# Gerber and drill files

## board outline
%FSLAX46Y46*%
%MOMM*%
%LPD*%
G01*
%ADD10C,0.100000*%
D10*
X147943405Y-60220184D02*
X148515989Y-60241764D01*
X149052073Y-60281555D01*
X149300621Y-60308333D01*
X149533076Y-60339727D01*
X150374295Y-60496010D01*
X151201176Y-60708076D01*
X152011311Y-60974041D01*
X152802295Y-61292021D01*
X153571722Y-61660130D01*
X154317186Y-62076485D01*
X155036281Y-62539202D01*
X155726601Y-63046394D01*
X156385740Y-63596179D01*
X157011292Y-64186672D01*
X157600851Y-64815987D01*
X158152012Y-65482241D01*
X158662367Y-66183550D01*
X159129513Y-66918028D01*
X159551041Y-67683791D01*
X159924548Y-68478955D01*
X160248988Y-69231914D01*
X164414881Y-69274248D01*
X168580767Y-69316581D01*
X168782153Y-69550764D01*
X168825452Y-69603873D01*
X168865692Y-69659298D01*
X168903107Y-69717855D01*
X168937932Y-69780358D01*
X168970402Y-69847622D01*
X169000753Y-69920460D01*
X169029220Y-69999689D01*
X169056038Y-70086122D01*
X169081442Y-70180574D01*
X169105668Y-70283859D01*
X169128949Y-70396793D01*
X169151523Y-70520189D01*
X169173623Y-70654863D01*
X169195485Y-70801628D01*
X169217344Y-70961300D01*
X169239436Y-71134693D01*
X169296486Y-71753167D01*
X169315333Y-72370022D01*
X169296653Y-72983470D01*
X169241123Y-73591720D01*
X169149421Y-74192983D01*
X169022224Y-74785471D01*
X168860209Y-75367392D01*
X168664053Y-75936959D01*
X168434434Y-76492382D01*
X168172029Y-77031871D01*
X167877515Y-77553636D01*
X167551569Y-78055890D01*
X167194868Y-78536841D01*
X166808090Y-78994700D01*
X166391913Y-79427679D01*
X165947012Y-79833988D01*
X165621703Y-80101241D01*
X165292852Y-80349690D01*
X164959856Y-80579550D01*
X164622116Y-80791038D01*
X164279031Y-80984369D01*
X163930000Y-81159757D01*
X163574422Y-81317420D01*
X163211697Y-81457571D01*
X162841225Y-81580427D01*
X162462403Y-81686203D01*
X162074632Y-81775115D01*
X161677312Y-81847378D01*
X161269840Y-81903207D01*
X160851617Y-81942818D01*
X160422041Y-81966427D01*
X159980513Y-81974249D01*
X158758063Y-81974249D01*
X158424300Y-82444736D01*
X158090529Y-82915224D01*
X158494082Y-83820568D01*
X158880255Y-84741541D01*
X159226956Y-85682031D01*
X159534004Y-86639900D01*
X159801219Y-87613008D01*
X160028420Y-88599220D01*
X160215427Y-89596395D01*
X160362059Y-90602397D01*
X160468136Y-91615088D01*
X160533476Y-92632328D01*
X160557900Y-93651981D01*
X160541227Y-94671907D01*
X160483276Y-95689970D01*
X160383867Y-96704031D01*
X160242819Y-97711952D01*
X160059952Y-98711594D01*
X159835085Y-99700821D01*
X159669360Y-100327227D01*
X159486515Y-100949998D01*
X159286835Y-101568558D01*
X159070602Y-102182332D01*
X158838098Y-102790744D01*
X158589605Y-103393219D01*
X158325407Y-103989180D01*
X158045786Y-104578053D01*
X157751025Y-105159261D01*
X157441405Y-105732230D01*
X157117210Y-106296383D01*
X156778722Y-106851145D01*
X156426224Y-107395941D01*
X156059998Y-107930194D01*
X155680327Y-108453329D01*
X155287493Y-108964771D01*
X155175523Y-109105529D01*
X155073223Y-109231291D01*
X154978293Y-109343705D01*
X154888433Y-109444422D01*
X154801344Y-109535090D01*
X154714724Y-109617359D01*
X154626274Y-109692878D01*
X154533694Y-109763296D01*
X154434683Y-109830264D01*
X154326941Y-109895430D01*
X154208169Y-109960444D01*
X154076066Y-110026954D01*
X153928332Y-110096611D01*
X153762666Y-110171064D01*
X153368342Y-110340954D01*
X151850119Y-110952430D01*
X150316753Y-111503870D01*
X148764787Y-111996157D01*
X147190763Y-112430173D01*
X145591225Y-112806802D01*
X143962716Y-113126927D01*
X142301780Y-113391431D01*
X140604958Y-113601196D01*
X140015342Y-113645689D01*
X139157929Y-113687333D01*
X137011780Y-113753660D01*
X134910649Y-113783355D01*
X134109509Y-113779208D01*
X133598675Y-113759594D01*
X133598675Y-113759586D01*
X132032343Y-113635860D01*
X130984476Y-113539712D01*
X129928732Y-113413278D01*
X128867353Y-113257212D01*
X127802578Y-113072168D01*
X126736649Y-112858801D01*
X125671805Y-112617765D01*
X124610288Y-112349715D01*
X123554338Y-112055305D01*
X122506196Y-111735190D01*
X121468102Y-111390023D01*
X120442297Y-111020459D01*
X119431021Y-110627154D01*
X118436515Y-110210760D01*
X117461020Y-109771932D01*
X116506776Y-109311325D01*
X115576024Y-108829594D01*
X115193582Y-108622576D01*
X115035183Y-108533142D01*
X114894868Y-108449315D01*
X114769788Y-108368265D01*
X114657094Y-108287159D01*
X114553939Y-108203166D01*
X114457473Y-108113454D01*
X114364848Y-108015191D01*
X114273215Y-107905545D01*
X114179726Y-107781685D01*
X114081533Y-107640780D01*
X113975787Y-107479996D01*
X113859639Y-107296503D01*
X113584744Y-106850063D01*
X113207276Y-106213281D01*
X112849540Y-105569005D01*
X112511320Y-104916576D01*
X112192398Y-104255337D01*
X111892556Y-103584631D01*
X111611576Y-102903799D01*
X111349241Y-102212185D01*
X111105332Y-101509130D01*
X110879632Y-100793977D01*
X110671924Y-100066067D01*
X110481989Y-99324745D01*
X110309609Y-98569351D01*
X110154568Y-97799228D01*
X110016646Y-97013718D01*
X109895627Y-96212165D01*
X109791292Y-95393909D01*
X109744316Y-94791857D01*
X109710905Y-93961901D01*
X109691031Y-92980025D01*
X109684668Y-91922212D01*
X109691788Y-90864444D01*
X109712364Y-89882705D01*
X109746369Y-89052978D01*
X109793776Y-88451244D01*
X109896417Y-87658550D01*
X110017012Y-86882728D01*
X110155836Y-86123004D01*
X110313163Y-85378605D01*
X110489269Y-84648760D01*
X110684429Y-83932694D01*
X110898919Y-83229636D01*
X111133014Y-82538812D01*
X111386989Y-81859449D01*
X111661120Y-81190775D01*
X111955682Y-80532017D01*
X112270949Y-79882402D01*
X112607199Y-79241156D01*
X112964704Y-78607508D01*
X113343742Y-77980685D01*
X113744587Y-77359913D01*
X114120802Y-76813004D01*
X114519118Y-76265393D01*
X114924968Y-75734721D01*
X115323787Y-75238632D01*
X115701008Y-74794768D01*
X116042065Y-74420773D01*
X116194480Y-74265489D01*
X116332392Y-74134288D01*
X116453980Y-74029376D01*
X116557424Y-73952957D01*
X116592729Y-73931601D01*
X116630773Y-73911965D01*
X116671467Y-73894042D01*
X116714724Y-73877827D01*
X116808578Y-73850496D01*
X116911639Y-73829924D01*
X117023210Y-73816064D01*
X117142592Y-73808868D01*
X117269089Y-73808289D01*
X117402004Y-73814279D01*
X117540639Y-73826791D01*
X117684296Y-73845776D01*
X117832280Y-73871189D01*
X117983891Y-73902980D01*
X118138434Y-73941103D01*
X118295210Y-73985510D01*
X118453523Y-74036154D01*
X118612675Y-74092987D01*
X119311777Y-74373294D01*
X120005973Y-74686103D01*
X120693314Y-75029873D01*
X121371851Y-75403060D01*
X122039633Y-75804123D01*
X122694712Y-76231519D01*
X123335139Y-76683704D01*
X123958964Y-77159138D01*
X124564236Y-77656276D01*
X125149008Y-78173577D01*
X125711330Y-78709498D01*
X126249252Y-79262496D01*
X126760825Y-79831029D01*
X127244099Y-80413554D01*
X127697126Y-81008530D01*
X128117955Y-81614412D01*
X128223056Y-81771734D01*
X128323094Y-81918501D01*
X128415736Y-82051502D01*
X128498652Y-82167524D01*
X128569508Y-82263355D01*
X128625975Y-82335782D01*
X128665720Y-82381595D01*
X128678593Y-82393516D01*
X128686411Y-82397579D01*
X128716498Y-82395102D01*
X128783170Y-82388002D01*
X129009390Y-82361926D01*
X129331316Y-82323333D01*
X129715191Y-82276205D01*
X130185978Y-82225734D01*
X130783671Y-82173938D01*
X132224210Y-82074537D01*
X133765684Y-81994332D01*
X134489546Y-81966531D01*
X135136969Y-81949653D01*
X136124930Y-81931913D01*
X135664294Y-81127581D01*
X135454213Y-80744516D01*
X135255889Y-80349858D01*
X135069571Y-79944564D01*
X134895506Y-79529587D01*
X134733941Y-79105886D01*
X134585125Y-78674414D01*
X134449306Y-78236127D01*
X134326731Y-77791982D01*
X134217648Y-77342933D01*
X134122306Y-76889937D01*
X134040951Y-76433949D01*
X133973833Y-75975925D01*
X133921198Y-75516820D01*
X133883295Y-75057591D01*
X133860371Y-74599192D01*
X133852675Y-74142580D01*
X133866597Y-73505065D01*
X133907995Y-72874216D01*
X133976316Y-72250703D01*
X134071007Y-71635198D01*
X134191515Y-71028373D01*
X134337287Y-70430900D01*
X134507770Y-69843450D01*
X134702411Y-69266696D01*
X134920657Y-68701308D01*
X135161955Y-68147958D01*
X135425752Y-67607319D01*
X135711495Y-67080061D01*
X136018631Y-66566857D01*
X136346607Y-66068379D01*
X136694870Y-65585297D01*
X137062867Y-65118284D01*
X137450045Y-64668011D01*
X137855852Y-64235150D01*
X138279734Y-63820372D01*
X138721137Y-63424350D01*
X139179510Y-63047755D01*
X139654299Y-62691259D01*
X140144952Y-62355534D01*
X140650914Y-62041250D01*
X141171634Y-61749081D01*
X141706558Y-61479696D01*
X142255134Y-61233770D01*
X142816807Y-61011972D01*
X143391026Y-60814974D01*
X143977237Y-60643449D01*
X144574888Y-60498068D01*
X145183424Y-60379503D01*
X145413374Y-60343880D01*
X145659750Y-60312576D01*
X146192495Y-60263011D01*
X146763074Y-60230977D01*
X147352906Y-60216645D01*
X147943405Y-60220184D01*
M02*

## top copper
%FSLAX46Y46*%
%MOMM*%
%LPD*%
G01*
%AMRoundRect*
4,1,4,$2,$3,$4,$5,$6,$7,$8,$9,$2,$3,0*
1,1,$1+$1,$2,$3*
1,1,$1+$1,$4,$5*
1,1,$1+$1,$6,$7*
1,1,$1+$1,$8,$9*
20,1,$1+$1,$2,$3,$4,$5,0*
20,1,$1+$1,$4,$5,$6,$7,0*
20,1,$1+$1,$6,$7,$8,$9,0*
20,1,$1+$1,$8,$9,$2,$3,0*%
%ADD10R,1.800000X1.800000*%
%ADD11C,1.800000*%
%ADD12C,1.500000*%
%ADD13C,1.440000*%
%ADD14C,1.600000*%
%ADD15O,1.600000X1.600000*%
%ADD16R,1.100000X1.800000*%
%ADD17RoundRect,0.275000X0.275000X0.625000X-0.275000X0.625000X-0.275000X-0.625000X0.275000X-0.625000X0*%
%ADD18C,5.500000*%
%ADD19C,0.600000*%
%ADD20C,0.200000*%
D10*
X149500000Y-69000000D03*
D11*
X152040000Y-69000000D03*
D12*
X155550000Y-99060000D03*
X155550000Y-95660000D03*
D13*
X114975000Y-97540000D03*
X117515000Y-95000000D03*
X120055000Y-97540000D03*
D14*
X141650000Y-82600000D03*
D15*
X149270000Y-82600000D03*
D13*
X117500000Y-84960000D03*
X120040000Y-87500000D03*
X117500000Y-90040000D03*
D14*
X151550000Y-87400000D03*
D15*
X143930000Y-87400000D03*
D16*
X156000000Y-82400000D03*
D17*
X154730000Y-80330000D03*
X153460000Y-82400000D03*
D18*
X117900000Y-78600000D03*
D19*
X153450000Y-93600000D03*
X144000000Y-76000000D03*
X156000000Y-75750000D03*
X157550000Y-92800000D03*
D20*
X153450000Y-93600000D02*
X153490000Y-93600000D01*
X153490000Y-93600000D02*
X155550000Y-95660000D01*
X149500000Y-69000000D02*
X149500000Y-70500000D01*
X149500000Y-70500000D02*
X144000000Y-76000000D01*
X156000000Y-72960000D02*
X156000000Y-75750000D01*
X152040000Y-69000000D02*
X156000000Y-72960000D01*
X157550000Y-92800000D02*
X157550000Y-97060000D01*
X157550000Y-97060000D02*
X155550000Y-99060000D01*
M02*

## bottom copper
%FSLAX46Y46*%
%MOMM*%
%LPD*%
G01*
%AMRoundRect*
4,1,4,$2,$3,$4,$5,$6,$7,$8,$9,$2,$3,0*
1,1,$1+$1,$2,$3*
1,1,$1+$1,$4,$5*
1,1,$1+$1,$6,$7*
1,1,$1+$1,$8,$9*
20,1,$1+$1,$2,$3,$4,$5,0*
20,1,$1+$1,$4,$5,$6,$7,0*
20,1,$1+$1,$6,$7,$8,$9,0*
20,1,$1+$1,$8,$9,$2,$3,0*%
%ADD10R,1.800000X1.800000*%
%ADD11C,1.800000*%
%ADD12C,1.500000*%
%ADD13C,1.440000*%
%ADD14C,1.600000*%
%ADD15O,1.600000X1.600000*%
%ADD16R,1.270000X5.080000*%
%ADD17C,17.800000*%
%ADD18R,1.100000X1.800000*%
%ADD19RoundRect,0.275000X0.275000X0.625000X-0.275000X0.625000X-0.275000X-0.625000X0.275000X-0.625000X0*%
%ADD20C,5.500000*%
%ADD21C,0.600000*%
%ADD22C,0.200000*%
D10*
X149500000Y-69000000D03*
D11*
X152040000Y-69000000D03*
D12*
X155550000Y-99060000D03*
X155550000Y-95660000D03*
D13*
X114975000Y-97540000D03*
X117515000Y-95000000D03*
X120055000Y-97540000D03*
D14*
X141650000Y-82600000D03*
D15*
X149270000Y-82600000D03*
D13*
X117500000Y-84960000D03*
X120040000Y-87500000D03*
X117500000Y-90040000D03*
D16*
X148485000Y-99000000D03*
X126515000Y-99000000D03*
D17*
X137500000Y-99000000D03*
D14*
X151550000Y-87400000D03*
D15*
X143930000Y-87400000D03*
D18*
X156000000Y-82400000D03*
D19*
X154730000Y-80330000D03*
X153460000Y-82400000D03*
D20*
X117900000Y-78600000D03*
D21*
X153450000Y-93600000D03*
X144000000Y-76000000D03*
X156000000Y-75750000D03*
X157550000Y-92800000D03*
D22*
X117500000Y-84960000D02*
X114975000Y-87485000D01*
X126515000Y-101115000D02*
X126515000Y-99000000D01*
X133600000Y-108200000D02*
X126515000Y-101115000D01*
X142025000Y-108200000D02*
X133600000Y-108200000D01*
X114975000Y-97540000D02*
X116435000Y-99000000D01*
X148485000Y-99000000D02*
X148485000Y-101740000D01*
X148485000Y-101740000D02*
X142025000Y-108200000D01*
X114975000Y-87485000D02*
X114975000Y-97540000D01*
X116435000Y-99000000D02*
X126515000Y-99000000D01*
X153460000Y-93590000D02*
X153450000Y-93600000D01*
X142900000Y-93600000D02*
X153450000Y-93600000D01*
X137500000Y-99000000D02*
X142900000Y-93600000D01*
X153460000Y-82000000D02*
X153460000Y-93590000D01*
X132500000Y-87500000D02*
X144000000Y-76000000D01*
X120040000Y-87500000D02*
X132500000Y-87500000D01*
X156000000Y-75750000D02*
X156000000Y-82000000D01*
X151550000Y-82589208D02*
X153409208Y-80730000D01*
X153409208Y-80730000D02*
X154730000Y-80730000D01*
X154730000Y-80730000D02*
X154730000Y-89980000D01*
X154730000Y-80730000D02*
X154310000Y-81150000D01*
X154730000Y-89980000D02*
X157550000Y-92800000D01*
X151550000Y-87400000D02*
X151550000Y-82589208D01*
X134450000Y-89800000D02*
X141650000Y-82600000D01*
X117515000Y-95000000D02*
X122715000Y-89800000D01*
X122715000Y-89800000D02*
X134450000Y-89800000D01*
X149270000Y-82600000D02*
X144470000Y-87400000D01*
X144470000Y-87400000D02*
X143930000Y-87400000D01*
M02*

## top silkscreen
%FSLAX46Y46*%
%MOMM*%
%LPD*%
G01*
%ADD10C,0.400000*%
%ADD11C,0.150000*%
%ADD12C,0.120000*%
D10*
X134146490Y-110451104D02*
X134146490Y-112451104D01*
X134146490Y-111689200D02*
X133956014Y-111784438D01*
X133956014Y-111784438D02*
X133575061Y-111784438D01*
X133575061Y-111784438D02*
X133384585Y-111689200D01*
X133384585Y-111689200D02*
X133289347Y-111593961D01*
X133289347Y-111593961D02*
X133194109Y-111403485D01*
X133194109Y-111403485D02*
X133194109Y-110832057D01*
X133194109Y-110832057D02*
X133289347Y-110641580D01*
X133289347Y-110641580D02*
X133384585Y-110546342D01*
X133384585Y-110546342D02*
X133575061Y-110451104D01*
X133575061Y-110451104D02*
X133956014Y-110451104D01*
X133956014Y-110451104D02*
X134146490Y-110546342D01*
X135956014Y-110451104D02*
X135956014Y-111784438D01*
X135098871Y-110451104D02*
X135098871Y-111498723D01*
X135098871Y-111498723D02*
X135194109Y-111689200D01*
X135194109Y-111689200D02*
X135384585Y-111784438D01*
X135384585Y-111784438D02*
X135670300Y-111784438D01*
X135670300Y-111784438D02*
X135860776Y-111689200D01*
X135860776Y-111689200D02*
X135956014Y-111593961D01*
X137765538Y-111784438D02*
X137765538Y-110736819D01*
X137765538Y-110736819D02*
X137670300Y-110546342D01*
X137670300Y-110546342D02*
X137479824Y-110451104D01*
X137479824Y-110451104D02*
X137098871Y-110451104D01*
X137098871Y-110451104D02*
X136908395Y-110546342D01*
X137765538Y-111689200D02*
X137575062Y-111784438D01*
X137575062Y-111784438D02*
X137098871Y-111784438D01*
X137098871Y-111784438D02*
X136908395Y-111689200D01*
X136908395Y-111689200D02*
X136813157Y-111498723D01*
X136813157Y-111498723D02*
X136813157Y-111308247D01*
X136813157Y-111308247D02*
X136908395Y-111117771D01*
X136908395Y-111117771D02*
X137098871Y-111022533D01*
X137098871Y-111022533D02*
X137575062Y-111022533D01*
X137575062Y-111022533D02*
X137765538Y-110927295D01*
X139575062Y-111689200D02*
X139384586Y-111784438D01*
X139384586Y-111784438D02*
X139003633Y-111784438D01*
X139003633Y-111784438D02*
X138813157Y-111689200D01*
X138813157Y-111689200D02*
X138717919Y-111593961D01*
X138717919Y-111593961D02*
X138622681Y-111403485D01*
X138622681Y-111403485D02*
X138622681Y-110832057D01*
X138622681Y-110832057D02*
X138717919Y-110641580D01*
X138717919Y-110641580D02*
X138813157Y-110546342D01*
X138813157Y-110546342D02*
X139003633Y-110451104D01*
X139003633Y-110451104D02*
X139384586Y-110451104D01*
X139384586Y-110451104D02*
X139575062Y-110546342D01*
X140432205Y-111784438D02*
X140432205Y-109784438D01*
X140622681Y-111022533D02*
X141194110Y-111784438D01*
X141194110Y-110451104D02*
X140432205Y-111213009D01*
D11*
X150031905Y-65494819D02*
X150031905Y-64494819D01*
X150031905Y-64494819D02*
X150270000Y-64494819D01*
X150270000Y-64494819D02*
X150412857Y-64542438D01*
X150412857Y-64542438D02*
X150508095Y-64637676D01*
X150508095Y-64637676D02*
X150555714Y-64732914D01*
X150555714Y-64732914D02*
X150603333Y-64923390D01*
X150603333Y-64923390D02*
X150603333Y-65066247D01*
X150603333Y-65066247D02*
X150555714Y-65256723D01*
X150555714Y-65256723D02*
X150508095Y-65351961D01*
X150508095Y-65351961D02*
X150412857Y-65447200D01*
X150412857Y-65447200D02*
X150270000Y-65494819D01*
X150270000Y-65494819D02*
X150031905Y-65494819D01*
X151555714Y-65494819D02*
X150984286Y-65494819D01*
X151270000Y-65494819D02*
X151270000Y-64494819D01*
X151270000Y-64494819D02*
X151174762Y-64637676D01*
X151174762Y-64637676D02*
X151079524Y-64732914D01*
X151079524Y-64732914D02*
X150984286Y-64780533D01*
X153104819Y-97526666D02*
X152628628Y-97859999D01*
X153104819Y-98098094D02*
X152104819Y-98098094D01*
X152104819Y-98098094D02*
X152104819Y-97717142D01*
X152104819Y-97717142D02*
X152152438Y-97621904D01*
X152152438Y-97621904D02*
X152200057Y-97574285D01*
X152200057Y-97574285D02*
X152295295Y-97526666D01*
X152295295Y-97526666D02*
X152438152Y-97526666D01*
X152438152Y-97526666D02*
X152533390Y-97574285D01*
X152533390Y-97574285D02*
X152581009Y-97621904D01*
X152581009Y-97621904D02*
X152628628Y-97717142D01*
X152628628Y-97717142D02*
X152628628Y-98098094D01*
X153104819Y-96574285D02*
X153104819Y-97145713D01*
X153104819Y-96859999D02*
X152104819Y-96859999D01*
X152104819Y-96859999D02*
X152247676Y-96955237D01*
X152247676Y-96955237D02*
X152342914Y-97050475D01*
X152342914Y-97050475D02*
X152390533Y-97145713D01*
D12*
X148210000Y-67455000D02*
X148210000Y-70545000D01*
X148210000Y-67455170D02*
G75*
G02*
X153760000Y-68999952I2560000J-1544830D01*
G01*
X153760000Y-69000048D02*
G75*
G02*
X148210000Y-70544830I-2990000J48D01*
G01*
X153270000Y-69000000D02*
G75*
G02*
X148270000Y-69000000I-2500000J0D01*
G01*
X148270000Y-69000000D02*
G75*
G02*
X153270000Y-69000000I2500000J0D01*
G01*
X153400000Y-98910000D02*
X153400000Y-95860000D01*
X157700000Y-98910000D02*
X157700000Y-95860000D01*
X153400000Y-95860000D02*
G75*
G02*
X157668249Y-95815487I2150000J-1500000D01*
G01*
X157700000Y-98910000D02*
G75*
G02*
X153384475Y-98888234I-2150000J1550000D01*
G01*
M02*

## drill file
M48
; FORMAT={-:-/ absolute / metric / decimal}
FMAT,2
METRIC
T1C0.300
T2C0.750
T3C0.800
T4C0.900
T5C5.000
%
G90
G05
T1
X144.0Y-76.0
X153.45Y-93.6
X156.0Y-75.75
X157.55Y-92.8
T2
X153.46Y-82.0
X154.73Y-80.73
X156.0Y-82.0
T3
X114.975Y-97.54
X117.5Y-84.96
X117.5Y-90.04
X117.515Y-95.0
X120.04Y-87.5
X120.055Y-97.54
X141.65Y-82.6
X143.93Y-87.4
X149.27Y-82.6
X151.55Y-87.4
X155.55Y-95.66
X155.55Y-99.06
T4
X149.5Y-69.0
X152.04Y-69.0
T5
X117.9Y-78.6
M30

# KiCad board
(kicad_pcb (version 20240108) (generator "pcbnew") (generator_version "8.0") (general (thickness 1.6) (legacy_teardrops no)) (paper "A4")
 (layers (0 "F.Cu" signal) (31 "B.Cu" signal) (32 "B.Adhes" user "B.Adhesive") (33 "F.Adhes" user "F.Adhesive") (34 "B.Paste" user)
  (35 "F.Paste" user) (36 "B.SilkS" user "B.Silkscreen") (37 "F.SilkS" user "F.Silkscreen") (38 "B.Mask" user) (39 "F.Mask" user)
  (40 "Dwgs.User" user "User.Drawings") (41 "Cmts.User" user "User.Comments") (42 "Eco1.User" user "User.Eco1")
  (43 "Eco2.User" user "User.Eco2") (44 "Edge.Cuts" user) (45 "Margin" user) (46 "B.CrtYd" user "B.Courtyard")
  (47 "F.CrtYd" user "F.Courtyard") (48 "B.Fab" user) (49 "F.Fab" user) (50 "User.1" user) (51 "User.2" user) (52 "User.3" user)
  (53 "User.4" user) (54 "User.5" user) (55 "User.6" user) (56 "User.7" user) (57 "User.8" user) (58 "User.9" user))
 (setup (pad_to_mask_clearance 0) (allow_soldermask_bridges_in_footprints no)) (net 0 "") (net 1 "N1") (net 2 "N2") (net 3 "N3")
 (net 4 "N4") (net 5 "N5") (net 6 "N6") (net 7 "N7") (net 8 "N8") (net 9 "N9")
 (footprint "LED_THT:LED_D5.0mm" (layer "F.Cu") (at 149.5 69)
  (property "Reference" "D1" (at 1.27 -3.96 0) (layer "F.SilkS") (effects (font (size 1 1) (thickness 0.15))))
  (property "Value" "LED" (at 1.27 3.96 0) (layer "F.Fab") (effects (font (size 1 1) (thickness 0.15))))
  (fp_line (start -1.29 -1.545) (end -1.29 1.545) (stroke (width 0.12) (type solid)) (layer "F.SilkS"))
  (fp_arc (start -1.29 -1.54483) (mid 2.071756 -2.880501) (end 4.26 -0.000048) (stroke (width 0.12) (type solid)) (layer "F.SilkS"))
  (fp_arc (start 4.26 0.000048) (mid 2.071756 2.880501) (end -1.29 1.54483) (stroke (width 0.12) (type solid)) (layer "F.SilkS"))
  (fp_circle (center 1.27 0) (end 3.77 0) (stroke (width 0.12) (type solid)) (fill none) (layer "F.SilkS"))
  (pad "1" thru_hole rect (at 0 0) (size 1.8 1.8) (drill 0.9) (layers "*.Cu" "*.Mask") (remove_unused_layers no) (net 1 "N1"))
  (pad "2" thru_hole circle (at 2.54 0) (size 1.8 1.8) (drill 0.9) (layers "*.Cu" "*.Mask") (remove_unused_layers no) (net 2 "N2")))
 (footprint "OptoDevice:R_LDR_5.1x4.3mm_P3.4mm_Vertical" (layer "F.Cu") (at 155.55 99.06 90)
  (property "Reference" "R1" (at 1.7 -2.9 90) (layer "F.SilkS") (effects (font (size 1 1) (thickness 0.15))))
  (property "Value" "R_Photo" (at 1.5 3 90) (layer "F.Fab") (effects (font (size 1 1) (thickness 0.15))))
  (fp_line (start 0.15 -2.15) (end 3.2 -2.15) (stroke (width 0.12) (type solid)) (layer "F.SilkS"))
  (fp_line (start 0.15 2.15) (end 3.2 2.15) (stroke (width 0.12) (type solid)) (layer "F.SilkS"))
  (fp_arc (start 3.2 -2.15) (mid 4.321403 -0.027338) (end 3.244513 2.118249) (stroke (width 0.12) (type solid)) (layer "F.SilkS"))
  (fp_arc (start 0.15 2.15) (mid -0.950438 -0.013368) (end 0.171766 -2.165525) (stroke (width 0.12) (type solid)) (layer "F.SilkS"))
  (pad "1" thru_hole circle (at 0 0 90) (size 1.5 1.5) (drill 0.8) (layers "*.Cu" "*.Mask") (remove_unused_layers no) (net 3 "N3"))
  (pad "2" thru_hole circle (at 3.4 0 90) (size 1.5 1.5) (drill 0.8) (layers "*.Cu" "*.Mask") (remove_unused_layers no) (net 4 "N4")))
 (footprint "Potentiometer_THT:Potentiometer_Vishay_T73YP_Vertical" (layer "B.Cu") (at 114.975 97.54 90)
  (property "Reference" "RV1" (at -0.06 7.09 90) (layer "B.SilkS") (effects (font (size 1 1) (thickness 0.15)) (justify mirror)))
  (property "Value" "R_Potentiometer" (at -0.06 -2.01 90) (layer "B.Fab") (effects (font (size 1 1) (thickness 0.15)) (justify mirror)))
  (pad "1" thru_hole circle (at 0 0 90) (size 1.44 1.44) (drill 0.8) (layers "*.Cu" "*.Mask") (remove_unused_layers no) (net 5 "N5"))
  (pad "2" thru_hole circle (at 2.54 2.54 90) (size 1.44 1.44) (drill 0.8) (layers "*.Cu" "*.Mask") (remove_unused_layers no) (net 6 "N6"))
  (pad "3" thru_hole circle (at 0 5.08 90) (size 1.44 1.44) (drill 0.8) (layers "*.Cu" "*.Mask") (remove_unused_layers no) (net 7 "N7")))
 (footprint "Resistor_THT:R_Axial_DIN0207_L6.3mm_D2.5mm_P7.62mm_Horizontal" (layer "B.Cu") (at 141.65 82.6)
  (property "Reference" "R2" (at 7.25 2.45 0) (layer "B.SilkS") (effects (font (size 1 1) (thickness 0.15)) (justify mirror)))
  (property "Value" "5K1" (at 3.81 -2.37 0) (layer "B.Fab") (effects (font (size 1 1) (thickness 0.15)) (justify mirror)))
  (pad "1" thru_hole circle (at 0 0) (size 1.6 1.6) (drill 0.8) (layers "*.Cu" "*.Mask") (remove_unused_layers no) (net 6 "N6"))
  (pad "2" thru_hole oval (at 7.62 0) (size 1.6 1.6) (drill 0.8) (layers "*.Cu" "*.Mask") (remove_unused_layers no) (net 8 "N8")))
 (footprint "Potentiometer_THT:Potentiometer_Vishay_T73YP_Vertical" (layer "B.Cu") (at 117.5 84.96)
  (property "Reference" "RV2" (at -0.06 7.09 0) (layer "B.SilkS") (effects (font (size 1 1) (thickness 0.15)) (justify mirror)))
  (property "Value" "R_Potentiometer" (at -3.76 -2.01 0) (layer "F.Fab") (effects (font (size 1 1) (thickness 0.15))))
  (pad "1" thru_hole circle (at 0 0) (size 1.44 1.44) (drill 0.8) (layers "*.Cu" "*.Mask") (remove_unused_layers no) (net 5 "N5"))
  (pad "2" thru_hole circle (at 2.54 2.54) (size 1.44 1.44) (drill 0.8) (layers "*.Cu" "*.Mask") (remove_unused_layers no) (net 1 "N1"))
  (pad "3" thru_hole circle (at 0 5.08) (size 1.44 1.44) (drill 0.8) (layers "*.Cu" "*.Mask") (remove_unused_layers no) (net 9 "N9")))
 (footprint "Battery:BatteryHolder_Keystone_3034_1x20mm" (layer "B.Cu") (at 137.5 99 180)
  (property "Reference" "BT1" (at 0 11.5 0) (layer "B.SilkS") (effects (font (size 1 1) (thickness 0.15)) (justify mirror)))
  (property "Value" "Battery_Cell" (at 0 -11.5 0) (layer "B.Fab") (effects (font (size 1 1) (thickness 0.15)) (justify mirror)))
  (pad "1" smd rect (at -10.985 0 180) (size 1.27 5.08) (layers "B.Cu" "B.Paste" "B.Mask") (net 5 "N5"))
  (pad "1" smd rect (at 10.985 0 180) (size 1.27 5.08) (layers "B.Cu" "B.Paste" "B.Mask") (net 5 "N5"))
  (pad "2" smd circle (at 0 0 180) (size 17.8 17.8) (layers "B.Cu" "B.Mask") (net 4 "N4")))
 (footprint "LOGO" (layer "B.Cu") (at 143.276488 74.088629 180)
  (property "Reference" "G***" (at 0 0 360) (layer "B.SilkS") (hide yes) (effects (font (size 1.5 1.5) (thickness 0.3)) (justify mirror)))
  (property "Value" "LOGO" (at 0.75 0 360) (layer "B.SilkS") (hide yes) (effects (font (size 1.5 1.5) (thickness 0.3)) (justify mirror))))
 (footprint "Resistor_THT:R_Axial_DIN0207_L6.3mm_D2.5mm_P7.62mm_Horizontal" (layer "B.Cu") (at 151.55 87.4 180)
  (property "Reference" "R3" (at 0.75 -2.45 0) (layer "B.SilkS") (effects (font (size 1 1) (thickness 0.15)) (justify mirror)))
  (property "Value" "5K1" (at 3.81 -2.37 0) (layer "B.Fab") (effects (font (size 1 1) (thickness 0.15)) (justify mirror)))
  (pad "1" thru_hole circle (at 0 0 180) (size 1.6 1.6) (drill 0.8) (layers "*.Cu" "*.Mask") (remove_unused_layers no) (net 3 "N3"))
  (pad "2" thru_hole oval (at 7.62 0 180) (size 1.6 1.6) (drill 0.8) (layers "*.Cu" "*.Mask") (remove_unused_layers no) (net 8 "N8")))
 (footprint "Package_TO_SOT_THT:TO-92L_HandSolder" (layer "B.Cu") (at 156 82 180)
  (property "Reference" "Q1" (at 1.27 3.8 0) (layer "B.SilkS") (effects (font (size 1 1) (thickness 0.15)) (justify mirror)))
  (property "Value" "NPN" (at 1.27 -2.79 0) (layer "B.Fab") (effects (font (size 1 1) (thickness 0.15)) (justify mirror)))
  (pad "1" thru_hole rect (at 0 0 180) (size 1.1 1.8) (drill 0.75 (offset 0 -0.4)) (layers "*.Cu" "*.Mask") (remove_unused_layers no)
   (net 2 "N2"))
  (pad "2" thru_hole roundrect (at 1.27 1.27 180) (size 1.1 1.8) (drill 0.75 (offset 0 0.4)) (layers "*.Cu" "*.Mask")
   (remove_unused_layers no) (roundrect_rratio 0.25) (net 3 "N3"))
  (pad "3" thru_hole roundrect (at 2.54 0 180) (size 1.1 1.8) (drill 0.75 (offset 0 -0.4)) (layers "*.Cu" "*.Mask")
   (remove_unused_layers no) (roundrect_rratio 0.25) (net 4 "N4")))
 (gr_poly
  (pts (xy 147.943405 60.220184) (xy 148.515989 60.241764) (xy 149.052073 60.281555) (xy 149.300621 60.308333) (xy 149.533076 60.339727)
   (xy 150.374295 60.49601) (xy 151.201176 60.708076) (xy 152.011311 60.974041) (xy 152.802295 61.292021) (xy 153.571722 61.66013)
   (xy 154.317186 62.076485) (xy 155.036281 62.539202) (xy 155.726601 63.046394) (xy 156.38574 63.596179) (xy 157.011292 64.186672)
   (xy 157.600851 64.815987) (xy 158.152012 65.482241) (xy 158.662367 66.18355) (xy 159.129513 66.918028) (xy 159.551041 67.683791)
   (xy 159.924548 68.478955) (xy 160.248988 69.231914) (xy 164.414881 69.274248) (xy 168.580767 69.316581) (xy 168.782153 69.550764)
   (xy 168.825452 69.603873) (xy 168.865692 69.659298) (xy 168.903107 69.717855) (xy 168.937932 69.780358) (xy 168.970402 69.847622)
   (xy 169.000753 69.92046) (xy 169.02922 69.999689) (xy 169.056038 70.086122) (xy 169.081442 70.180574) (xy 169.105668 70.283859)
   (xy 169.128949 70.396793) (xy 169.151523 70.520189) (xy 169.173623 70.654863) (xy 169.195485 70.801628) (xy 169.217344 70.9613)
   (xy 169.239436 71.134693) (xy 169.296486 71.753167) (xy 169.315333 72.370022) (xy 169.296653 72.98347) (xy 169.241123 73.59172)
   (xy 169.149421 74.192983) (xy 169.022224 74.785471) (xy 168.860209 75.367392) (xy 168.664053 75.936959) (xy 168.434434 76.492382)
   (xy 168.172029 77.031871) (xy 167.877515 77.553636) (xy 167.551569 78.05589) (xy 167.194868 78.536841) (xy 166.80809 78.9947)
   (xy 166.391913 79.427679) (xy 165.947012 79.833988) (xy 165.621703 80.101241) (xy 165.292852 80.34969) (xy 164.959856 80.57955)
   (xy 164.622116 80.791038) (xy 164.279031 80.984369) (xy 163.93 81.159757) (xy 163.574422 81.31742) (xy 163.211697 81.457571)
   (xy 162.841225 81.580427) (xy 162.462403 81.686203) (xy 162.074632 81.775115) (xy 161.677312 81.847378) (xy 161.26984 81.903207)
   (xy 160.851617 81.942818) (xy 160.422041 81.966427) (xy 159.980513 81.974249) (xy 158.758063 81.974249) (xy 158.4243 82.444736)
   (xy 158.090529 82.915224) (xy 158.494082 83.820568) (xy 158.880255 84.741541) (xy 159.226956 85.682031) (xy 159.534004 86.6399)
   (xy 159.801219 87.613008) (xy 160.02842 88.59922) (xy 160.215427 89.596395) (xy 160.362059 90.602397) (xy 160.468136 91.615088)
   (xy 160.533476 92.632328) (xy 160.5579 93.651981) (xy 160.541227 94.671907) (xy 160.483276 95.68997) (xy 160.383867 96.704031)
   (xy 160.242819 97.711952) (xy 160.059952 98.711594) (xy 159.835085 99.700821) (xy 159.66936 100.327227) (xy 159.486515 100.949998)
   (xy 159.286835 101.568558) (xy 159.070602 102.182332) (xy 158.838098 102.790744) (xy 158.589605 103.393219) (xy 158.325407 103.98918)
   (xy 158.045786 104.578053) (xy 157.751025 105.159261) (xy 157.441405 105.73223) (xy 157.11721 106.296383) (xy 156.778722 106.851145)
   (xy 156.426224 107.395941) (xy 156.059998 107.930194) (xy 155.680327 108.453329) (xy 155.287493 108.964771) (xy 155.175523 109.105529)
   (xy 155.073223 109.231291) (xy 154.978293 109.343705) (xy 154.888433 109.444422) (xy 154.801344 109.53509) (xy 154.714724 109.617359)
   (xy 154.626274 109.692878) (xy 154.533694 109.763296) (xy 154.434683 109.830264) (xy 154.326941 109.89543) (xy 154.208169 109.960444)
   (xy 154.076066 110.026954) (xy 153.928332 110.096611) (xy 153.762666 110.171064) (xy 153.368342 110.340954) (xy 151.850119 110.95243)
   (xy 150.316753 111.50387) (xy 148.764787 111.996157) (xy 147.190763 112.430173) (xy 145.591225 112.806802) (xy 143.962716 113.126927)
   (xy 142.30178 113.391431) (xy 140.604958 113.601196) (xy 140.015342 113.645689) (xy 139.157929 113.687333) (xy 137.01178 113.75366)
   (xy 134.910649 113.783355) (xy 134.109509 113.779208) (xy 133.598675 113.759594) (xy 133.598675 113.759586) (xy 132.032343 113.63586)
   (xy 130.984476 113.539712) (xy 129.928732 113.413278) (xy 128.867353 113.257212) (xy 127.802578 113.072168) (xy 126.736649 112.858801)
   (xy 125.671805 112.617765) (xy 124.610288 112.349715) (xy 123.554338 112.055305) (xy 122.506196 111.73519) (xy 121.468102 111.390023)
   (xy 120.442297 111.020459) (xy 119.431021 110.627154) (xy 118.436515 110.21076) (xy 117.46102 109.771932) (xy 116.506776 109.311325)
   (xy 115.576024 108.829594) (xy 115.193582 108.622576) (xy 115.035183 108.533142) (xy 114.894868 108.449315) (xy 114.769788 108.368265)
   (xy 114.657094 108.287159) (xy 114.553939 108.203166) (xy 114.457473 108.113454) (xy 114.364848 108.015191) (xy 114.273215 107.905545)
   (xy 114.179726 107.781685) (xy 114.081533 107.64078) (xy 113.975787 107.479996) (xy 113.859639 107.296503) (xy 113.584744 106.850063)
   (xy 113.207276 106.213281) (xy 112.84954 105.569005) (xy 112.51132 104.916576) (xy 112.192398 104.255337) (xy 111.892556 103.584631)
   (xy 111.611576 102.903799) (xy 111.349241 102.212185) (xy 111.105332 101.50913) (xy 110.879632 100.793977) (xy 110.671924 100.066067)
   (xy 110.481989 99.324745) (xy 110.309609 98.569351) (xy 110.154568 97.799228) (xy 110.016646 97.013718) (xy 109.895627 96.212165)
   (xy 109.791292 95.393909) (xy 109.744316 94.791857) (xy 109.710905 93.961901) (xy 109.691031 92.980025) (xy 109.684668 91.922212)
   (xy 109.691788 90.864444) (xy 109.712364 89.882705) (xy 109.746369 89.052978) (xy 109.793776 88.451244) (xy 109.896417 87.65855)
   (xy 110.017012 86.882728) (xy 110.155836 86.123004) (xy 110.313163 85.378605) (xy 110.489269 84.64876) (xy 110.684429 83.932694)
   (xy 110.898919 83.229636) (xy 111.133014 82.538812) (xy 111.386989 81.859449) (xy 111.66112 81.190775) (xy 111.955682 80.532017)
   (xy 112.270949 79.882402) (xy 112.607199 79.241156) (xy 112.964704 78.607508) (xy 113.343742 77.980685) (xy 113.744587 77.359913)
   (xy 114.120802 76.813004) (xy 114.519118 76.265393) (xy 114.924968 75.734721) (xy 115.323787 75.238632) (xy 115.701008 74.794768)
   (xy 116.042065 74.420773) (xy 116.19448 74.265489) (xy 116.332392 74.134288) (xy 116.45398 74.029376) (xy 116.557424 73.952957)
   (xy 116.592729 73.931601) (xy 116.630773 73.911965) (xy 116.671467 73.894042) (xy 116.714724 73.877827) (xy 116.808578 73.850496)
   (xy 116.911639 73.829924) (xy 117.02321 73.816064) (xy 117.142592 73.808868) (xy 117.269089 73.808289) (xy 117.402004 73.814279)
   (xy 117.540639 73.826791) (xy 117.684296 73.845776) (xy 117.83228 73.871189) (xy 117.983891 73.90298) (xy 118.138434 73.941103)
   (xy 118.29521 73.98551) (xy 118.453523 74.036154) (xy 118.612675 74.092987) (xy 119.311777 74.373294) (xy 120.005973 74.686103)
   (xy 120.693314 75.029873) (xy 121.371851 75.40306) (xy 122.039633 75.804123) (xy 122.694712 76.231519) (xy 123.335139 76.683704)
   (xy 123.958964 77.159138) (xy 124.564236 77.656276) (xy 125.149008 78.173577) (xy 125.71133 78.709498) (xy 126.249252 79.262496)
   (xy 126.760825 79.831029) (xy 127.244099 80.413554) (xy 127.697126 81.00853) (xy 128.117955 81.614412) (xy 128.223056 81.771734)
   (xy 128.323094 81.918501) (xy 128.415736 82.051502) (xy 128.498652 82.167524) (xy 128.569508 82.263355) (xy 128.625975 82.335782)
   (xy 128.66572 82.381595) (xy 128.678593 82.393516) (xy 128.686411 82.397579) (xy 128.716498 82.395102) (xy 128.78317 82.388002)
   (xy 129.00939 82.361926) (xy 129.331316 82.323333) (xy 129.715191 82.276205) (xy 130.185978 82.225734) (xy 130.783671 82.173938)
   (xy 132.22421 82.074537) (xy 133.765684 81.994332) (xy 134.489546 81.966531) (xy 135.136969 81.949653) (xy 136.12493 81.931913)
   (xy 135.664294 81.127581) (xy 135.454213 80.744516) (xy 135.255889 80.349858) (xy 135.069571 79.944564) (xy 134.895506 79.529587)
   (xy 134.733941 79.105886) (xy 134.585125 78.674414) (xy 134.449306 78.236127) (xy 134.326731 77.791982) (xy 134.217648 77.342933)
   (xy 134.122306 76.889937) (xy 134.040951 76.433949) (xy 133.973833 75.975925) (xy 133.921198 75.51682) (xy 133.883295 75.057591)
   (xy 133.860371 74.599192) (xy 133.852675 74.14258) (xy 133.866597 73.505065) (xy 133.907995 72.874216) (xy 133.976316 72.250703)
   (xy 134.071007 71.635198) (xy 134.191515 71.028373) (xy 134.337287 70.4309) (xy 134.50777 69.84345) (xy 134.702411 69.266696)
   (xy 134.920657 68.701308) (xy 135.161955 68.147958) (xy 135.425752 67.607319) (xy 135.711495 67.080061) (xy 136.018631 66.566857)
   (xy 136.346607 66.068379) (xy 136.69487 65.585297) (xy 137.062867 65.118284) (xy 137.450045 64.668011) (xy 137.855852 64.23515)
   (xy 138.279734 63.820372) (xy 138.721137 63.42435) (xy 139.17951 63.047755) (xy 139.654299 62.691259) (xy 140.144952 62.355534)
   (xy 140.650914 62.04125) (xy 141.171634 61.749081) (xy 141.706558 61.479696) (xy 142.255134 61.23377) (xy 142.816807 61.011972)
   (xy 143.391026 60.814974) (xy 143.977237 60.643449) (xy 144.574888 60.498068) (xy 145.183424 60.379503) (xy 145.413374 60.34388)
   (xy 145.65975 60.312576) (xy 146.192495 60.263011) (xy 146.763074 60.230977) (xy 147.352906 60.216645))
  (stroke (width 0.1) (type solid)) (fill none) (layer "Edge.Cuts"))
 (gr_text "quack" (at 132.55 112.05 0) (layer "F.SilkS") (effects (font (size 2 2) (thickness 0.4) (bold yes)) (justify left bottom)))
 (via (at 117.9 78.6) (size 5.5) (drill 5) (layers "F.Cu" "B.Cu") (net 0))
 (segment (start 117.5 84.96) (end 114.975 87.485) (width 0.2) (layer "B.Cu") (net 5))
 (segment (start 126.515 101.115) (end 126.515 99) (width 0.2) (layer "B.Cu") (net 5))
 (segment (start 133.6 108.2) (end 126.515 101.115) (width 0.2) (layer "B.Cu") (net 5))
 (segment (start 142.025 108.2) (end 133.6 108.2) (width 0.2) (layer "B.Cu") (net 5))
 (segment (start 114.975 97.54) (end 116.435 99) (width 0.2) (layer "B.Cu") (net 5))
 (segment (start 148.485 99) (end 148.485 101.74) (width 0.2) (layer "B.Cu") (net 5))
 (segment (start 148.485 101.74) (end 142.025 108.2) (width 0.2) (layer "B.Cu") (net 5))
 (segment (start 114.975 87.485) (end 114.975 97.54) (width 0.2) (layer "B.Cu") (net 5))
 (segment (start 116.435 99) (end 126.515 99) (width 0.2) (layer "B.Cu") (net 5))
 (segment (start 153.45 93.6) (end 153.49 93.6) (width 0.2) (layer "F.Cu") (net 4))
 (segment (start 153.49 93.6) (end 155.55 95.66) (width 0.2) (layer "F.Cu") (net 4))
 (via (at 153.45 93.6) (size 0.6) (drill 0.3) (layers "F.Cu" "B.Cu") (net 4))
 (segment (start 153.46 93.59) (end 153.45 93.6) (width 0.2) (layer "B.Cu") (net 4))
 (segment (start 142.9 93.6) (end 153.45 93.6) (width 0.2) (layer "B.Cu") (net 4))
 (segment (start 137.5 99) (end 142.9 93.6) (width 0.2) (layer "B.Cu") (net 4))
 (segment (start 153.46 82) (end 153.46 93.59) (width 0.2) (layer "B.Cu") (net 4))
 (segment (start 149.5 69) (end 149.5 70.5) (width 0.2) (layer "F.Cu") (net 1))
 (segment (start 149.5 70.5) (end 144 76) (width 0.2) (layer "F.Cu") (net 1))
 (via (at 144 76) (size 0.6) (drill 0.3) (layers "F.Cu" "B.Cu") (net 1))
 (segment (start 132.5 87.5) (end 144 76) (width 0.2) (layer "B.Cu") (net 1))
 (segment (start 120.04 87.5) (end 132.5 87.5) (width 0.2) (layer "B.Cu") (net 1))
 (segment (start 156 72.96) (end 156 75.75) (width 0.2) (layer "F.Cu") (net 2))
 (segment (start 152.04 69) (end 156 72.96) (width 0.2) (layer "F.Cu") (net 2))
 (via (at 156 75.75) (size 0.6) (drill 0.3) (layers "F.Cu" "B.Cu") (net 2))
 (segment (start 156 75.75) (end 156 82) (width 0.2) (layer "B.Cu") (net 2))
 (segment (start 157.55 92.8) (end 157.55 97.06) (width 0.2) (layer "F.Cu") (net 3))
 (segment (start 157.55 97.06) (end 155.55 99.06) (width 0.2) (layer "F.Cu") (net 3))
 (via (at 157.55 92.8) (size 0.6) (drill 0.3) (layers "F.Cu" "B.Cu") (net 3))
 (segment (start 151.55 82.589208) (end 153.409208 80.73) (width 0.2) (layer "B.Cu") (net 3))
 (segment (start 153.409208 80.73) (end 154.73 80.73) (width 0.2) (layer "B.Cu") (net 3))
 (segment (start 154.73 80.73) (end 154.73 89.98) (width 0.2) (layer "B.Cu") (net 3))
 (segment (start 154.73 80.73) (end 154.31 81.15) (width 0.2) (layer "B.Cu") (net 3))
 (segment (start 154.73 89.98) (end 157.55 92.8) (width 0.2) (layer "B.Cu") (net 3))
 (segment (start 151.55 87.4) (end 151.55 82.589208) (width 0.2) (layer "B.Cu") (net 3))
 (segment (start 134.45 89.8) (end 141.65 82.6) (width 0.2) (layer "B.Cu") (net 6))
 (segment (start 117.515 95) (end 122.715 89.8) (width 0.2) (layer "B.Cu") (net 6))
 (segment (start 122.715 89.8) (end 134.45 89.8) (width 0.2) (layer "B.Cu") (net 6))
 (segment (start 149.27 82.6) (end 144.47 87.4) (width 0.2) (layer "B.Cu") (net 8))
 (segment (start 144.47 87.4) (end 143.93 87.4) (width 0.2) (layer "B.Cu") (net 8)))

